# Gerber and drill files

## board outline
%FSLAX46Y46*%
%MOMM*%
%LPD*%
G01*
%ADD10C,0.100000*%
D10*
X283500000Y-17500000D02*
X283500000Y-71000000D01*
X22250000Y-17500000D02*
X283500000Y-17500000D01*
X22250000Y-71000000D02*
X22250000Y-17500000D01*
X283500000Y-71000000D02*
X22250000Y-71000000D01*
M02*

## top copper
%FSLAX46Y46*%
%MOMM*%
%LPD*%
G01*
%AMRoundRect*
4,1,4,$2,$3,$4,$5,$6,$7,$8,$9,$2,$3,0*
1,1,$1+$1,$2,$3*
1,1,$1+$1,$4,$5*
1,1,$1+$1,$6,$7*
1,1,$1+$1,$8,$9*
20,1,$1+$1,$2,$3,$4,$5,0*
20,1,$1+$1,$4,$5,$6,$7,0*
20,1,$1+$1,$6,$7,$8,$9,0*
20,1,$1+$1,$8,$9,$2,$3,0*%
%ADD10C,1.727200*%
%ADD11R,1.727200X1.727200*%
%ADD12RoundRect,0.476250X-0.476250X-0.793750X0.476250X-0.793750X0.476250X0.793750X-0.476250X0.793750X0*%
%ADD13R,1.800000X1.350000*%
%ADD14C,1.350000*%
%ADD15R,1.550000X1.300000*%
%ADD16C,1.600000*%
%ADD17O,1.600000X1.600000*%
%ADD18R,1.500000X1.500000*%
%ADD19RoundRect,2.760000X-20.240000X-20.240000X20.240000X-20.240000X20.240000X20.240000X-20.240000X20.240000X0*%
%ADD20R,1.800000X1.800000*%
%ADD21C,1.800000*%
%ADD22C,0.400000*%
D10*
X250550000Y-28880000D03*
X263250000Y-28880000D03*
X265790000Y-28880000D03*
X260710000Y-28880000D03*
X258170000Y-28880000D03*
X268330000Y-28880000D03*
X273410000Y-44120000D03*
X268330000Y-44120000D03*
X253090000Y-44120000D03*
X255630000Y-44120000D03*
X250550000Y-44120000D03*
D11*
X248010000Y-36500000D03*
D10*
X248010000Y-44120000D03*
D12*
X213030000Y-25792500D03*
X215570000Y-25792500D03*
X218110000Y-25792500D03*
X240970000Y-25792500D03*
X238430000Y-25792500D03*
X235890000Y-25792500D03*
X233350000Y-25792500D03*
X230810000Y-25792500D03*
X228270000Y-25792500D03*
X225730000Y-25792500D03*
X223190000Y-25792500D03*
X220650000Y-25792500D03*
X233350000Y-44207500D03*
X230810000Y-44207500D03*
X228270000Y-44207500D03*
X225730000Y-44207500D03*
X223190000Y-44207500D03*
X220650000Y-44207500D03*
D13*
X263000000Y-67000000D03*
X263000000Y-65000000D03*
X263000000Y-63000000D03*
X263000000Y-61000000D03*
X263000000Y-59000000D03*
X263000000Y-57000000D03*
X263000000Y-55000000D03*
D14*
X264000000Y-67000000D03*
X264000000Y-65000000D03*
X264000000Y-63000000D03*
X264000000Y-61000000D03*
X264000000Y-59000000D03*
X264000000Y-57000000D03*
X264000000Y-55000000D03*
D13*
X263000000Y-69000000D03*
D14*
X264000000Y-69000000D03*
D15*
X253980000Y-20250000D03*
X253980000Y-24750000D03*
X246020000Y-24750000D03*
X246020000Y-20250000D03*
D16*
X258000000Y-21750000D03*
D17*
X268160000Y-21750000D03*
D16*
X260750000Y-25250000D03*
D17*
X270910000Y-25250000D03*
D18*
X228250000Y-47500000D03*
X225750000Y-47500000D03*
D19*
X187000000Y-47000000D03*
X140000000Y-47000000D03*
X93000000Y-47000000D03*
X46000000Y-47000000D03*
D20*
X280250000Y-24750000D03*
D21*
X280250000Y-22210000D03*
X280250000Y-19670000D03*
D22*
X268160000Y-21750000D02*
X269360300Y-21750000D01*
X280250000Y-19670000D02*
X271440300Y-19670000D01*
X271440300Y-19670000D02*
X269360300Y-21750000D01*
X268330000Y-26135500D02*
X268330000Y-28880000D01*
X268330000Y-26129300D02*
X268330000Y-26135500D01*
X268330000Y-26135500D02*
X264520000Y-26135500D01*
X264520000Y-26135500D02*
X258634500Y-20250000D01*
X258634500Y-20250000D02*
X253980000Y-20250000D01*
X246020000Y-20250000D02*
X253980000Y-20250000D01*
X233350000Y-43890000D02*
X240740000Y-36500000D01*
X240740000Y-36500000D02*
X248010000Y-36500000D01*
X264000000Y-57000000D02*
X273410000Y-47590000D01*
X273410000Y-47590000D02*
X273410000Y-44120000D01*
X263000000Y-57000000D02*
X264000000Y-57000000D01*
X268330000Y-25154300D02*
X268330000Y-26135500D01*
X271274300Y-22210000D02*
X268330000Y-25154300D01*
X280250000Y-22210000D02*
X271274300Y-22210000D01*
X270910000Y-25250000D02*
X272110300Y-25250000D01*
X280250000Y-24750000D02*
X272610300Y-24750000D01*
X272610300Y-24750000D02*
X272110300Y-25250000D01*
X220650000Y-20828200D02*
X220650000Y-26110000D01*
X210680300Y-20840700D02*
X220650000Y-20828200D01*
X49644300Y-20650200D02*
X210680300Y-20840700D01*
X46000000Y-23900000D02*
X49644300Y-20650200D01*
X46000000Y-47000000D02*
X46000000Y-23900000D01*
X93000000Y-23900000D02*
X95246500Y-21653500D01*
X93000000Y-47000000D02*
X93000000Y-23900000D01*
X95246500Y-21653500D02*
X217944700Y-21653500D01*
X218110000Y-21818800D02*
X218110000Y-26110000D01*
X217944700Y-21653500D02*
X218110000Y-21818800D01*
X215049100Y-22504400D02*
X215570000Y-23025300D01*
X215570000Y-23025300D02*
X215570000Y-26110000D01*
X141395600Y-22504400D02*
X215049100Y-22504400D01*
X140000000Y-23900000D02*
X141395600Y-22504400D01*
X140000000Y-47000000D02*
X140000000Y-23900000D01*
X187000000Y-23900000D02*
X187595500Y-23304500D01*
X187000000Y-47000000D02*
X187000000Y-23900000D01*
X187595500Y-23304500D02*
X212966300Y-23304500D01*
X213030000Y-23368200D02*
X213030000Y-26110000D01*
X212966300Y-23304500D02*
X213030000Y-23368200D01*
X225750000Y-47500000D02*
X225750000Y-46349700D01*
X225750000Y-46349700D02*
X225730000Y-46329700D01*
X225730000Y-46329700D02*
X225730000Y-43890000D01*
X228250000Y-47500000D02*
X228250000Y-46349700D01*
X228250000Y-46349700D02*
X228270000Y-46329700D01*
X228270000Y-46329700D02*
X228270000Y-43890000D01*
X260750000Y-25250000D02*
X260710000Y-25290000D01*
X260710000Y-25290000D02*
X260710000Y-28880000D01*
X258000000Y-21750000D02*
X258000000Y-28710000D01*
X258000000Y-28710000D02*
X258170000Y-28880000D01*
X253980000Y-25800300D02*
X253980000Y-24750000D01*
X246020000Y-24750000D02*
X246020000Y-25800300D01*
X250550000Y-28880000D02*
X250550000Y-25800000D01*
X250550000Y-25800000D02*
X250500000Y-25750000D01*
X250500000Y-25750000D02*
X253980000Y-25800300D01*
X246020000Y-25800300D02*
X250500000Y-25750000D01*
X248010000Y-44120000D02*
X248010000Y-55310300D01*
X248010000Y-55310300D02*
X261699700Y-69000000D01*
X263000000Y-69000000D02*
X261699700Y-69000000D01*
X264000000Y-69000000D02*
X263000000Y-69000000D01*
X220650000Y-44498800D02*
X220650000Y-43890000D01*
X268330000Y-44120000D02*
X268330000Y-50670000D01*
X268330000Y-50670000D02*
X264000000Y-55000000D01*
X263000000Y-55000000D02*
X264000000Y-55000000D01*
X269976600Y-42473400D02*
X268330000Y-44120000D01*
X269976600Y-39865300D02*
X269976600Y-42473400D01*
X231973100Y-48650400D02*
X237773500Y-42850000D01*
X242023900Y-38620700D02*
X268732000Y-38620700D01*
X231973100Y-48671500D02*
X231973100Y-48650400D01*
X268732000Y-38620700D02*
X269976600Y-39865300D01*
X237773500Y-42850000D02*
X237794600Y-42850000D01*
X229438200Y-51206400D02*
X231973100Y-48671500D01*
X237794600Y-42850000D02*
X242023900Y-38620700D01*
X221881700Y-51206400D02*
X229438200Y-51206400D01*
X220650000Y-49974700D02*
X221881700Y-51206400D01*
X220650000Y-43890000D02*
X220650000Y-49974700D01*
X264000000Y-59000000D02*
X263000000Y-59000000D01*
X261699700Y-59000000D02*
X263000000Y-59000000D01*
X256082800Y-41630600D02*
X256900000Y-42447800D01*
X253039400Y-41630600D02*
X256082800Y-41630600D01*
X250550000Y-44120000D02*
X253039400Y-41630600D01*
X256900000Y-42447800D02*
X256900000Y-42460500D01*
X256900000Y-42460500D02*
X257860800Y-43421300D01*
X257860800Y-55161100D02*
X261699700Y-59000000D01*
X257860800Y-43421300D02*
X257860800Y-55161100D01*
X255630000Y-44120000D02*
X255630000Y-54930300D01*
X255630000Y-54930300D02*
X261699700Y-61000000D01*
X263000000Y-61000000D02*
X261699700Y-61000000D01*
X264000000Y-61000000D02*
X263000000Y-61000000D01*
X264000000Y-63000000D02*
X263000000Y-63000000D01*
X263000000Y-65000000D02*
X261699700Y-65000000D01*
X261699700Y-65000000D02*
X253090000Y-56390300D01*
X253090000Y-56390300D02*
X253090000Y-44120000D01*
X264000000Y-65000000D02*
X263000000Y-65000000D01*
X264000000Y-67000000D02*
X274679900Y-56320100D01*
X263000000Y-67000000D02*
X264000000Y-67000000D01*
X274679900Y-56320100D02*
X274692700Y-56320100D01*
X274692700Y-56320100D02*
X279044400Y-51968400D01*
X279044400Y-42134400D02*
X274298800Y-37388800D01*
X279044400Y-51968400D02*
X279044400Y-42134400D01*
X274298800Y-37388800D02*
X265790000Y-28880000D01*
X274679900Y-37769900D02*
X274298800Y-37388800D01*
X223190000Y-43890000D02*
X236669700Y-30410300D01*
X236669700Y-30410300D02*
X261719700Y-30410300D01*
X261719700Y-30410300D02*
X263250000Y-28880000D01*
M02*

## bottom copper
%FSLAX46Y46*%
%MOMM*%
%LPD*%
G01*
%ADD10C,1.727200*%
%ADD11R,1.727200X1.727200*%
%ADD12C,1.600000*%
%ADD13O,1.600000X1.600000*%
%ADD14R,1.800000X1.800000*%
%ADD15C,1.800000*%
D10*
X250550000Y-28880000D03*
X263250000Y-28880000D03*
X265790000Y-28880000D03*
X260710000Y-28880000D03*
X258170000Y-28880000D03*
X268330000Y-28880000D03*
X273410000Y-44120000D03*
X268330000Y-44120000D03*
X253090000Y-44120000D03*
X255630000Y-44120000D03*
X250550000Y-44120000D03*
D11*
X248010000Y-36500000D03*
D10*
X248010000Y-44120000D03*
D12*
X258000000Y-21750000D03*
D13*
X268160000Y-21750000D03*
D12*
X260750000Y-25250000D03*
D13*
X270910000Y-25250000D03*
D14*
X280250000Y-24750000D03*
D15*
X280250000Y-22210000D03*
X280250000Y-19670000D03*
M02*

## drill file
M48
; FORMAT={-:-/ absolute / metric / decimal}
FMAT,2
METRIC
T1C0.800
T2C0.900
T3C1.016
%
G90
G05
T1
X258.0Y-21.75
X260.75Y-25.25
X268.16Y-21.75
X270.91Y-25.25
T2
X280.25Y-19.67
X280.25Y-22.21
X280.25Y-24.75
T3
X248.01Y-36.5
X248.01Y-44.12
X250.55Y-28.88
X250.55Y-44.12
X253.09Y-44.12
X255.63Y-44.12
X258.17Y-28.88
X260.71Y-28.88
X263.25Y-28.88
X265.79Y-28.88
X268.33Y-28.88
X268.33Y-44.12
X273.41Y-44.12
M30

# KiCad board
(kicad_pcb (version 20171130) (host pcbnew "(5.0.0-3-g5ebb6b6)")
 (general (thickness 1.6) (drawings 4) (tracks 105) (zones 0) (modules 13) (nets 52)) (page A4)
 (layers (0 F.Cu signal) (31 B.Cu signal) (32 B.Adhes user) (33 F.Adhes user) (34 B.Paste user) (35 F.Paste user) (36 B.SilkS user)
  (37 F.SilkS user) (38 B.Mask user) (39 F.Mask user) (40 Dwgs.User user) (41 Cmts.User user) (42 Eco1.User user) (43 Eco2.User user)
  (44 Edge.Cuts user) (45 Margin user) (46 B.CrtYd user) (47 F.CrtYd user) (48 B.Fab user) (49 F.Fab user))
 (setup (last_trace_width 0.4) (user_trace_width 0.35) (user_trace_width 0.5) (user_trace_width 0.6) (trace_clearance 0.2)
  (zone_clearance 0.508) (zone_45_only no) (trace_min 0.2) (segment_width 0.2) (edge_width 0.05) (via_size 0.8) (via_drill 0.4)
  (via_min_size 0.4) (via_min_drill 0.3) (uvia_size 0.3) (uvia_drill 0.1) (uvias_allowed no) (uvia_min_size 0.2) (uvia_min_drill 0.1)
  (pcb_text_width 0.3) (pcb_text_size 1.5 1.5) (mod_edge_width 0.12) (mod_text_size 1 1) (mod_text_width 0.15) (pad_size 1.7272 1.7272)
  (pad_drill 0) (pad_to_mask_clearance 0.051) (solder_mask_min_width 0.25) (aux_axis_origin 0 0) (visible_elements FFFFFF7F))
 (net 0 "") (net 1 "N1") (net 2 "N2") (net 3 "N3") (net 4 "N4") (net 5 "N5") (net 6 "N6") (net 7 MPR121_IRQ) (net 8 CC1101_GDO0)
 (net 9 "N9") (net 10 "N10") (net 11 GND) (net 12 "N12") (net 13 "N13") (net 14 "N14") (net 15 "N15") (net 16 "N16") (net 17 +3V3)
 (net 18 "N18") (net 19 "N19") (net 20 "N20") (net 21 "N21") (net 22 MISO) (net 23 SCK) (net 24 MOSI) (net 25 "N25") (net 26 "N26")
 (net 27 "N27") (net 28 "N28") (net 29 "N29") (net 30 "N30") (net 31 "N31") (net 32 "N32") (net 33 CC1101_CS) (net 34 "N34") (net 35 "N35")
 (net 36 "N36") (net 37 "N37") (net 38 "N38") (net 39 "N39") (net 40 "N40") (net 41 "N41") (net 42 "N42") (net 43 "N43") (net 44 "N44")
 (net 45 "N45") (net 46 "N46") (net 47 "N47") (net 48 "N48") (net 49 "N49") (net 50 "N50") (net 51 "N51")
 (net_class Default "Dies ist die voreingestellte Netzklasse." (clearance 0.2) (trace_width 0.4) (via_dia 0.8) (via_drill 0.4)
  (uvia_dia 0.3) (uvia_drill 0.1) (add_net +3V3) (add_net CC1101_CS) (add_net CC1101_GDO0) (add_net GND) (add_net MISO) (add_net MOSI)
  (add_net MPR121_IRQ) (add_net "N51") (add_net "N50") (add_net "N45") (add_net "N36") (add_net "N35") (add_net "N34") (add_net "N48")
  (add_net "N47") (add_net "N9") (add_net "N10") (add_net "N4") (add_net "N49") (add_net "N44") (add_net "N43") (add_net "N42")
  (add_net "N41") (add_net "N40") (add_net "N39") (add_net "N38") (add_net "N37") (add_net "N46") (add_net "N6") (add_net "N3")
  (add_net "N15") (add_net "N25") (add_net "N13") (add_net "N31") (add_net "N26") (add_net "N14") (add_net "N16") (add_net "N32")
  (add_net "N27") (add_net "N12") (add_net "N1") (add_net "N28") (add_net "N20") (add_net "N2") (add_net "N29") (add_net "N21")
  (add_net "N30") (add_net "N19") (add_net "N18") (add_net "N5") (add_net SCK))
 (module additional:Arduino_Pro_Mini (layer F.Cu) (at 263.25 36.5 270)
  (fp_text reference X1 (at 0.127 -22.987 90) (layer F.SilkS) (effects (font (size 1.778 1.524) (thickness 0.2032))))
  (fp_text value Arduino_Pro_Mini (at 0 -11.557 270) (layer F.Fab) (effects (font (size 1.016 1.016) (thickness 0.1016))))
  (pad 4B connect circle (at 5.08 -1.27 270) (size 1.7272 1.7272) (layers F.Mask) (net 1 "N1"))
  (pad 5B connect circle (at 5.08 -3.81 270) (size 1.7272 1.7272) (layers F.Mask) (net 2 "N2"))
  (pad 12D connect circle (at -7.62 15.24 270) (size 1.7272 1.7272) (layers F.Mask) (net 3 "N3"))
  (pad 11D thru_hole circle (at -7.62 12.7 270) (size 1.7272 1.7272) (drill 1.016) (layers *.Cu *.Mask F.SilkS) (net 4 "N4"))
  (pad 9D connect circle (at -7.62 7.62 270) (size 1.7272 1.7272) (layers F.Mask) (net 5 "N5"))
  (pad 10D connect circle (at -7.62 10.16 270) (size 1.7272 1.7272) (layers F.Mask) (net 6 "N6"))
  (pad 6D thru_hole circle (at -7.62 0 270) (size 1.7272 1.7272) (drill 1.016) (layers *.Cu *.Mask F.SilkS) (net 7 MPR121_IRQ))
  (pad 5D thru_hole circle (at -7.62 -2.54 270) (size 1.7272 1.7272) (drill 1.016) (layers *.Cu *.Mask F.SilkS) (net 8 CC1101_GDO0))
  (pad 7D thru_hole circle (at -7.62 2.54 270) (size 1.7272 1.7272) (drill 1.016) (layers *.Cu *.Mask F.SilkS) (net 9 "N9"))
  (pad 8D thru_hole circle (at -7.62 5.08 270) (size 1.7272 1.7272) (drill 1.016) (layers *.Cu *.Mask F.SilkS) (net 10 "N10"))
  (pad 4D thru_hole circle (at -7.62 -5.08 270) (size 1.7272 1.7272) (drill 1.016) (layers *.Cu *.Mask F.SilkS) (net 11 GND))
  (pad 3D connect circle (at -7.62 -7.62 270) (size 1.7272 1.7272) (layers F.Mask) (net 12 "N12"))
  (pad 1D connect rect (at -7.62 -12.7 270) (size 1.7272 1.7272) (layers F.Mask) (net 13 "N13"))
  (pad 2D connect circle (at -7.62 -10.16 270) (size 1.7272 1.7272) (layers F.Mask) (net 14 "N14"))
  (pad 2A thru_hole circle (at 7.62 -10.16 270) (size 1.7272 1.7272) (drill 1.016) (layers *.Cu *.Mask F.SilkS) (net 11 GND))
  (pad 1A connect rect (at 7.62 -12.7 270) (size 1.7272 1.7272) (layers F.Mask) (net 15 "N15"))
  (pad 3A connect circle (at 7.62 -7.62 270) (size 1.7272 1.7272) (layers F.Mask) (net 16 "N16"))
  (pad 4A thru_hole circle (at 7.62 -5.08 270) (size 1.7272 1.7272) (drill 1.016) (layers *.Cu *.Mask F.SilkS) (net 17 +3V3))
  (pad 8A connect circle (at 7.62 5.08 270) (size 1.7272 1.7272) (layers F.Mask) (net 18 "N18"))
  (pad 7A connect circle (at 7.62 2.54 270) (size 1.7272 1.7272) (layers F.Mask) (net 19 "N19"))
  (pad 5A connect circle (at 7.62 -2.54 270) (size 1.7272 1.7272) (layers F.Mask) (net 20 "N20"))
  (pad 6A connect circle (at 7.62 0 270) (size 1.7272 1.7272) (layers F.Mask) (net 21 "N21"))
  (pad 10A thru_hole circle (at 7.62 10.16 270) (size 1.7272 1.7272) (drill 1.016) (layers *.Cu *.Mask F.SilkS) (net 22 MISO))
  (pad 9A thru_hole circle (at 7.62 7.62 270) (size 1.7272 1.7272) (drill 1.016) (layers *.Cu *.Mask F.SilkS) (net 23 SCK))
  (pad 11A thru_hole circle (at 7.62 12.7 270) (size 1.7272 1.7272) (drill 1.016) (layers *.Cu *.Mask F.SilkS) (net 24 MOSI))
  (pad 1C connect rect (at -6.35 -15.24 270) (size 1.7272 1.7272) (layers F.Mask) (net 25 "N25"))
  (pad 2C connect circle (at -3.81 -15.24 270) (size 1.7272 1.7272) (layers F.Mask) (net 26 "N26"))
  (pad 3C connect circle (at -1.27 -15.24 270) (size 1.7272 1.7272) (layers F.Mask) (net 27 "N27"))
  (pad 4C connect circle (at 1.27 -15.24 270) (size 1.7272 1.7272) (layers F.Mask) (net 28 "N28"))
  (pad 5C connect circle (at 3.81 -15.24 270) (size 1.7272 1.7272) (layers F.Mask) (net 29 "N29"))
  (pad 6C connect circle (at 6.35 -15.24 270) (size 1.7272 1.7272) (layers F.Mask) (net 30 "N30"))
  (pad 1B thru_hole rect (at 0 15.24 270) (size 1.7272 1.7272) (drill 1.016) (layers *.Cu *.Mask F.SilkS) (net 11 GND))
  (pad 2B connect circle (at 2.54 15.24 270) (size 1.7272 1.7272) (layers F.Mask) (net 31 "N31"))
  (pad 3B connect circle (at 5.08 15.24 270) (size 1.7272 1.7272) (layers F.Mask) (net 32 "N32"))
  (pad 12A thru_hole circle (at 7.62 15.24 270) (size 1.7272 1.7272) (drill 1.016) (layers *.Cu *.Mask F.SilkS) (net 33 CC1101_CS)))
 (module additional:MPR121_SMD (layer F.Cu) (at 227 35)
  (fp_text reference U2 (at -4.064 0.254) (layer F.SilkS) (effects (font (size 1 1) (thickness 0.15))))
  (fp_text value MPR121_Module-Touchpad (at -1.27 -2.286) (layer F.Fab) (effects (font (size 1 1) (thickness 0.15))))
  (pad 7 smd roundrect (at -13.97 -8.89) (size 1.905 2.54) (drill oval (offset 0 -0.3175)) (layers F.Cu F.Paste F.Mask)
   (roundrect_rratio 0.25) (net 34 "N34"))
  (pad 8 smd roundrect (at -11.43 -8.89) (size 1.905 2.54) (drill oval (offset 0 -0.3175)) (layers F.Cu F.Paste F.Mask)
   (roundrect_rratio 0.25) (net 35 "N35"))
  (pad 9 smd roundrect (at -8.89 -8.89) (size 1.905 2.54) (drill oval (offset 0 -0.3175)) (layers F.Cu F.Paste F.Mask)
   (roundrect_rratio 0.25) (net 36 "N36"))
  (pad 18 smd roundrect (at 13.97 -8.89) (size 1.905 2.54) (drill oval (offset 0 -0.3175)) (layers F.Cu F.Paste F.Mask)
   (roundrect_rratio 0.25) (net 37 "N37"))
  (pad 17 smd roundrect (at 11.43 -8.89) (size 1.905 2.54) (drill oval (offset 0 -0.3175)) (layers F.Cu F.Paste F.Mask)
   (roundrect_rratio 0.25) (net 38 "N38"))
  (pad 16 smd roundrect (at 8.89 -8.89) (size 1.905 2.54) (drill oval (offset 0 -0.3175)) (layers F.Cu F.Paste F.Mask)
   (roundrect_rratio 0.25) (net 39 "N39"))
  (pad 15 smd roundrect (at 6.35 -8.89) (size 1.905 2.54) (drill oval (offset 0 -0.3175)) (layers F.Cu F.Paste F.Mask)
   (roundrect_rratio 0.25) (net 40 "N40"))
  (pad 14 smd roundrect (at 3.81 -8.89) (size 1.905 2.54) (drill oval (offset 0 -0.3175)) (layers F.Cu F.Paste F.Mask)
   (roundrect_rratio 0.25) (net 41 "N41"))
  (pad 13 smd roundrect (at 1.27 -8.89) (size 1.905 2.54) (drill oval (offset 0 -0.3175)) (layers F.Cu F.Paste F.Mask)
   (roundrect_rratio 0.25) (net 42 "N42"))
  (pad 12 smd roundrect (at -1.27 -8.89) (size 1.905 2.54) (drill oval (offset 0 -0.3175)) (layers F.Cu F.Paste F.Mask)
   (roundrect_rratio 0.25) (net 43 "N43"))
  (pad 11 smd roundrect (at -3.81 -8.89) (size 1.905 2.54) (drill oval (offset 0 -0.3175)) (layers F.Cu F.Paste F.Mask)
   (roundrect_rratio 0.25) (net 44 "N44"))
  (pad 10 smd roundrect (at -6.35 -8.89) (size 1.905 2.54) (drill oval (offset 0 -0.3175)) (layers F.Cu F.Paste F.Mask)
   (roundrect_rratio 0.25) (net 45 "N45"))
  (pad 6 smd roundrect (at 6.35 8.89) (size 1.905 2.54) (drill oval (offset 0 0.3175)) (layers F.Cu F.Paste F.Mask) (roundrect_rratio 0.25)
   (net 11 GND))
  (pad 5 smd roundrect (at 3.81 8.89) (size 1.905 2.54) (drill oval (offset 0 0.3175)) (layers F.Cu F.Paste F.Mask) (roundrect_rratio 0.25)
   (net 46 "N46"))
  (pad 4 smd roundrect (at 1.27 8.89) (size 1.905 2.54) (drill oval (offset 0 0.3175)) (layers F.Cu F.Paste F.Mask) (roundrect_rratio 0.25)
   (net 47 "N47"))
  (pad 3 smd roundrect (at -1.27 8.89) (size 1.905 2.54) (drill oval (offset 0 0.3175)) (layers F.Cu F.Paste F.Mask) (roundrect_rratio 0.25)
   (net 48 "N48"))
  (pad 2 smd roundrect (at -3.81 8.89) (size 1.905 2.54) (drill oval (offset 0 0.3175)) (layers F.Cu F.Paste F.Mask) (roundrect_rratio 0.25)
   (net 7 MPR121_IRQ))
  (pad 1 smd roundrect (at -6.35 8.89) (size 1.905 2.54) (drill oval (offset 0 0.3175)) (layers F.Cu F.Paste F.Mask) (roundrect_rratio 0.25)
   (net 17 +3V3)))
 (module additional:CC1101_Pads (layer F.Cu) (at 261.5 53.5)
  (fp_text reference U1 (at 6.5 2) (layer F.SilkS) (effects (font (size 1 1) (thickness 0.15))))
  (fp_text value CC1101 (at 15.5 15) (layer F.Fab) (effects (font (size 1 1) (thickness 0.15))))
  (pad 7 connect rect (at 1.5 13.5) (size 1.8 1.35) (layers F.Cu F.Mask) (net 8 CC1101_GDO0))
  (pad 6 connect rect (at 1.5 11.5) (size 1.8 1.35) (layers F.Cu F.Mask) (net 22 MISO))
  (pad 5 connect rect (at 1.5 9.5) (size 1.8 1.35) (layers F.Cu F.Mask) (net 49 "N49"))
  (pad 4 connect rect (at 1.5 7.5) (size 1.8 1.35) (layers F.Cu F.Mask) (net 23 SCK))
  (pad 3 connect rect (at 1.5 5.5) (size 1.8 1.35) (layers F.Cu F.Mask) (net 24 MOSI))
  (pad 2 connect rect (at 1.5 3.5) (size 1.8 1.35) (layers F.Cu F.Mask) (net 11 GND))
  (pad 1 connect rect (at 1.5 1.5) (size 1.8 1.35) (layers F.Cu F.Mask) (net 17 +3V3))
  (pad 7 smd circle (at 2.5 13.5) (size 1.35 1.35) (layers F.Cu F.Paste F.Mask) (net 8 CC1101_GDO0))
  (pad 6 smd circle (at 2.5 11.5) (size 1.35 1.35) (layers F.Cu F.Paste F.Mask) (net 22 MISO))
  (pad 5 smd circle (at 2.5 9.5) (size 1.35 1.35) (layers F.Cu F.Paste F.Mask) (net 49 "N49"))
  (pad 4 smd circle (at 2.5 7.5) (size 1.35 1.35) (layers F.Cu F.Paste F.Mask) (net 23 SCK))
  (pad 3 smd circle (at 2.5 5.5) (size 1.35 1.35) (layers F.Cu F.Paste F.Mask) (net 24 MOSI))
  (pad 2 smd circle (at 2.5 3.5) (size 1.35 1.35) (layers F.Cu F.Paste F.Mask) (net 11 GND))
  (pad 1 smd circle (at 2.5 1.5) (size 1.35 1.35) (layers F.Cu F.Paste F.Mask) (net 17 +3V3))
  (pad 8 connect rect (at 1.5 15.5) (size 1.8 1.35) (layers F.Cu F.Mask) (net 33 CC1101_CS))
  (pad 8 smd circle (at 2.5 15.5) (size 1.35 1.35) (layers F.Cu F.Paste F.Mask) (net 33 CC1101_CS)))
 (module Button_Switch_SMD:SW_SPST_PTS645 (layer F.Cu) (at 250 22.5 180)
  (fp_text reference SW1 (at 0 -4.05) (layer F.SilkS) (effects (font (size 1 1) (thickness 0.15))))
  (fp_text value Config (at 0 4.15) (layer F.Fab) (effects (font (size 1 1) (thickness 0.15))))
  (pad 2 smd rect (at -3.98 2.25 180) (size 1.55 1.3) (layers F.Cu F.Paste F.Mask) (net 11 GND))
  (pad 1 smd rect (at -3.98 -2.25 180) (size 1.55 1.3) (layers F.Cu F.Paste F.Mask) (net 4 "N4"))
  (pad 1 smd rect (at 3.98 -2.25 180) (size 1.55 1.3) (layers F.Cu F.Paste F.Mask) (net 4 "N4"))
  (pad 2 smd rect (at 3.98 2.25 180) (size 1.55 1.3) (layers F.Cu F.Paste F.Mask) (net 11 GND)))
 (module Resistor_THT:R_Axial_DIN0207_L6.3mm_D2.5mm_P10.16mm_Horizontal (layer F.Cu) (at 258 21.75)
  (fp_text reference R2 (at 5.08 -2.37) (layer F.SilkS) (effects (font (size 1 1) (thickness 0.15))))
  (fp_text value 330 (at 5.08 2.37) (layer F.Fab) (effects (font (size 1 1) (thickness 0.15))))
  (pad 1 thru_hole circle (at 0 0) (size 1.6 1.6) (drill 0.8) (layers *.Cu *.Mask) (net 10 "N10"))
  (pad 2 thru_hole oval (at 10.16 0) (size 1.6 1.6) (drill 0.8) (layers *.Cu *.Mask) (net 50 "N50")))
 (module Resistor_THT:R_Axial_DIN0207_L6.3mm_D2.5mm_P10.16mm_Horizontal (layer F.Cu) (at 260.75 25.25)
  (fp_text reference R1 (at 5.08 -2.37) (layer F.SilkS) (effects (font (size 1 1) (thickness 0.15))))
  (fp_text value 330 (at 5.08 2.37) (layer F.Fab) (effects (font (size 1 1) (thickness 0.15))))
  (pad 1 thru_hole circle (at 0 0) (size 1.6 1.6) (drill 0.8) (layers *.Cu *.Mask) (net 9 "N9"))
  (pad 2 thru_hole oval (at 10.16 0) (size 1.6 1.6) (drill 0.8) (layers *.Cu *.Mask) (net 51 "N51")))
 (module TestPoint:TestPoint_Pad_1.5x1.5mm (layer F.Cu) (at 228.25 47.5)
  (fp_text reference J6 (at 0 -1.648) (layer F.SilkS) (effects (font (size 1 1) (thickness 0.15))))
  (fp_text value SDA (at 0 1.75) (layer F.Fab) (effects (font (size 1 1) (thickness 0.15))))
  (pad 1 smd rect (at 0 0) (size 1.5 1.5) (layers F.Cu F.Mask) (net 47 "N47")))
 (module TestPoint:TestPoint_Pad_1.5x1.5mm (layer F.Cu) (at 225.75 47.5)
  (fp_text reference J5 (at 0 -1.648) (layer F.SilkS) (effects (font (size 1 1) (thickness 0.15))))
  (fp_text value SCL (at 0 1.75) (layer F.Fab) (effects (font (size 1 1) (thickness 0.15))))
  (pad 1 smd rect (at 0 0) (size 1.5 1.5) (layers F.Cu F.Mask) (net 48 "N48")))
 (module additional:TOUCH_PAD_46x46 (layer F.Cu) (at 187 47)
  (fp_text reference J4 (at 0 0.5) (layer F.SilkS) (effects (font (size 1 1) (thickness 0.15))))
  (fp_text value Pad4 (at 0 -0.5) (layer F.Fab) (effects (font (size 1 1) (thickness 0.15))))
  (pad 1 smd roundrect (at 0 0) (size 46 46) (layers F.Cu) (roundrect_rratio 0.06) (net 34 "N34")))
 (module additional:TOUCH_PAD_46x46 (layer F.Cu) (at 140 47)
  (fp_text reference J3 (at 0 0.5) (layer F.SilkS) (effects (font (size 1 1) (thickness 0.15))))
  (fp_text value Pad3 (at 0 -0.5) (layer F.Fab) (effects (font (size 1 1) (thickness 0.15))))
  (pad 1 smd roundrect (at 0 0) (size 46 46) (layers F.Cu) (roundrect_rratio 0.06) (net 35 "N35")))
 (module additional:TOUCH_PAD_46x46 (layer F.Cu) (at 93 47)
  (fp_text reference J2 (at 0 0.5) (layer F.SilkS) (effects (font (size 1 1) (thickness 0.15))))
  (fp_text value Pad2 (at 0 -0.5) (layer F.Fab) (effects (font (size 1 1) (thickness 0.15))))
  (pad 1 smd roundrect (at 0 0) (size 46 46) (layers F.Cu) (roundrect_rratio 0.06) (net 36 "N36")))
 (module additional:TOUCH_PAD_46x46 (layer F.Cu) (at 46 47)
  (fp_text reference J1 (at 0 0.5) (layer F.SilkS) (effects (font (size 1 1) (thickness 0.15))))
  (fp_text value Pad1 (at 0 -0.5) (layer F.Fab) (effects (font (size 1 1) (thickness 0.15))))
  (pad 1 smd roundrect (at 0 0) (size 46 46) (layers F.Cu) (roundrect_rratio 0.06) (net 45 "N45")))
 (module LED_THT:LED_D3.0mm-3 (layer F.Cu) (at 280.25 24.75 90)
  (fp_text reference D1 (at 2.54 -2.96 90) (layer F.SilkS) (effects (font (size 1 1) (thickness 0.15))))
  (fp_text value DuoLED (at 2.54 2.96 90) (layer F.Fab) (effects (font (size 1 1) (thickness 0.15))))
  (pad 1 thru_hole rect (at 0 0 90) (size 1.8 1.8) (drill 0.9) (layers *.Cu *.Mask) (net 51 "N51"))
  (pad 2 thru_hole circle (at 2.54 0 90) (size 1.8 1.8) (drill 0.9) (layers *.Cu *.Mask) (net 11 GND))
  (pad 3 thru_hole circle (at 5.08 0 90) (size 1.8 1.8) (drill 0.9) (layers *.Cu *.Mask) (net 50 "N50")))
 (gr_line (start 283.5 17.5) (end 283.5 71) (layer Edge.Cuts) (width 0.1))
 (gr_line (start 22.25 17.5) (end 283.5 17.5) (layer Edge.Cuts) (width 0.1))
 (gr_line (start 22.25 71) (end 22.25 17.5) (layer Edge.Cuts) (width 0.1))
 (gr_line (start 283.5 71) (end 22.25 71) (layer Edge.Cuts) (width 0.1))
 (segment (start 268.16 21.75) (end 269.3603 21.75) (width 0.4) (layer F.Cu) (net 50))
 (segment (start 280.25 19.67) (end 271.4403 19.67) (width 0.4) (layer F.Cu) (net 50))
 (segment (start 271.4403 19.67) (end 269.3603 21.75) (width 0.4) (layer F.Cu) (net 50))
 (segment (start 268.33 26.1355) (end 268.33 28.88) (width 0.4) (layer F.Cu) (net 11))
 (segment (start 268.33 26.1293) (end 268.33 26.1355) (width 0.4) (layer F.Cu) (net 11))
 (segment (start 268.33 26.1355) (end 264.52 26.1355) (width 0.4) (layer F.Cu) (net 11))
 (segment (start 264.52 26.1355) (end 258.6345 20.25) (width 0.4) (layer F.Cu) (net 11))
 (segment (start 258.6345 20.25) (end 253.98 20.25) (width 0.4) (layer F.Cu) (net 11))
 (segment (start 246.02 20.25) (end 253.98 20.25) (width 0.4) (layer F.Cu) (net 11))
 (segment (start 233.35 43.89) (end 240.74 36.5) (width 0.4) (layer F.Cu) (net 11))
 (segment (start 240.74 36.5) (end 248.01 36.5) (width 0.4) (layer F.Cu) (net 11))
 (segment (start 264 57) (end 273.41 47.59) (width 0.4) (layer F.Cu) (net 11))
 (segment (start 273.41 47.59) (end 273.41 44.12) (width 0.4) (layer F.Cu) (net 11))
 (segment (start 263 57) (end 264 57) (width 0.4) (layer F.Cu) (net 11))
 (segment (start 268.33 25.1543) (end 268.33 26.1355) (width 0.4) (layer F.Cu) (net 11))
 (segment (start 271.2743 22.21) (end 268.33 25.1543) (width 0.4) (layer F.Cu) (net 11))
 (segment (start 280.25 22.21) (end 271.2743 22.21) (width 0.4) (layer F.Cu) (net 11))
 (segment (start 270.91 25.25) (end 272.1103 25.25) (width 0.4) (layer F.Cu) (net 51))
 (segment (start 280.25 24.75) (end 272.6103 24.75) (width 0.4) (layer F.Cu) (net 51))
 (segment (start 272.6103 24.75) (end 272.1103 25.25) (width 0.4) (layer F.Cu) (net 51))
 (segment (start 220.65 20.8282) (end 220.65 26.11) (width 0.4) (layer F.Cu) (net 45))
 (segment (start 210.6803 20.8407) (end 220.65 20.8282) (width 0.4) (layer F.Cu) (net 45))
 (segment (start 49.6443 20.6502) (end 210.6803 20.8407) (width 0.4) (layer F.Cu) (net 45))
 (segment (start 46 23.9) (end 49.6443 20.6502) (width 0.4) (layer F.Cu) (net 45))
 (segment (start 46 47) (end 46 23.9) (width 0.4) (layer F.Cu) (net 45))
 (segment (start 93 23.9) (end 95.2465 21.6535) (width 0.4) (layer F.Cu) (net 36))
 (segment (start 93 47) (end 93 23.9) (width 0.4) (layer F.Cu) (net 36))
 (segment (start 95.2465 21.6535) (end 217.9447 21.6535) (width 0.4) (layer F.Cu) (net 36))
 (segment (start 218.11 21.8188) (end 218.11 26.11) (width 0.4) (layer F.Cu) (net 36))
 (segment (start 217.9447 21.6535) (end 218.11 21.8188) (width 0.4) (layer F.Cu) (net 36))
 (segment (start 215.0491 22.5044) (end 215.57 23.0253) (width 0.4) (layer F.Cu) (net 35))
 (segment (start 215.57 23.0253) (end 215.57 26.11) (width 0.4) (layer F.Cu) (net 35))
 (segment (start 141.3956 22.5044) (end 215.0491 22.5044) (width 0.4) (layer F.Cu) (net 35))
 (segment (start 140 23.9) (end 141.3956 22.5044) (width 0.4) (layer F.Cu) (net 35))
 (segment (start 140 47) (end 140 23.9) (width 0.4) (layer F.Cu) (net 35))
 (segment (start 187 23.9) (end 187.5955 23.3045) (width 0.4) (layer F.Cu) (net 34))
 (segment (start 187 47) (end 187 23.9) (width 0.4) (layer F.Cu) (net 34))
 (segment (start 187.5955 23.3045) (end 212.9663 23.3045) (width 0.4) (layer F.Cu) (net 34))
 (segment (start 213.03 23.3682) (end 213.03 26.11) (width 0.4) (layer F.Cu) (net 34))
 (segment (start 212.9663 23.3045) (end 213.03 23.3682) (width 0.4) (layer F.Cu) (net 34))
 (segment (start 225.75 47.5) (end 225.75 46.3497) (width 0.4) (layer F.Cu) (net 48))
 (segment (start 225.75 46.3497) (end 225.73 46.3297) (width 0.4) (layer F.Cu) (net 48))
 (segment (start 225.73 46.3297) (end 225.73 43.89) (width 0.4) (layer F.Cu) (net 48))
 (segment (start 228.25 47.5) (end 228.25 46.3497) (width 0.4) (layer F.Cu) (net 47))
 (segment (start 228.25 46.3497) (end 228.27 46.3297) (width 0.4) (layer F.Cu) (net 47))
 (segment (start 228.27 46.3297) (end 228.27 43.89) (width 0.4) (layer F.Cu) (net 47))
 (segment (start 260.75 25.25) (end 260.71 25.29) (width 0.4) (layer F.Cu) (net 9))
 (segment (start 260.71 25.29) (end 260.71 28.88) (width 0.4) (layer F.Cu) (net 9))
 (segment (start 258 21.75) (end 258 28.71) (width 0.4) (layer F.Cu) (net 10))
 (segment (start 258 28.71) (end 258.17 28.88) (width 0.4) (layer F.Cu) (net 10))
 (segment (start 253.98 25.8003) (end 253.98 24.75) (width 0.4) (layer F.Cu) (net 4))
 (segment (start 246.02 24.75) (end 246.02 25.8003) (width 0.4) (layer F.Cu) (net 4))
 (segment (start 250.55 28.88) (end 250.55 25.8) (width 0.4) (layer F.Cu) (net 4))
 (segment (start 250.55 25.8) (end 250.5 25.75) (width 0.4) (layer F.Cu) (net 4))
 (segment (start 250.5 25.75) (end 253.98 25.8003) (width 0.4) (layer F.Cu) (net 4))
 (segment (start 246.02 25.8003) (end 250.5 25.75) (width 0.4) (layer F.Cu) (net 4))
 (segment (start 248.01 44.12) (end 248.01 55.3103) (width 0.4) (layer F.Cu) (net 33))
 (segment (start 248.01 55.3103) (end 261.6997 69) (width 0.4) (layer F.Cu) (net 33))
 (segment (start 263 69) (end 261.6997 69) (width 0.4) (layer F.Cu) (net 33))
 (segment (start 264 69) (end 263 69) (width 0.4) (layer F.Cu) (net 33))
 (segment (start 220.65 44.4988) (end 220.65 43.89) (width 0.4) (layer F.Cu) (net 17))
 (segment (start 268.33 44.12) (end 268.33 50.67) (width 0.4) (layer F.Cu) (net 17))
 (segment (start 268.33 50.67) (end 264 55) (width 0.4) (layer F.Cu) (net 17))
 (segment (start 263 55) (end 264 55) (width 0.4) (layer F.Cu) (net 17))
 (segment (start 269.9766 42.4734) (end 268.33 44.12) (width 0.4) (layer F.Cu) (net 17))
 (segment (start 269.9766 39.8653) (end 269.9766 42.4734) (width 0.4) (layer F.Cu) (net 17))
 (segment (start 231.9731 48.6504) (end 237.7735 42.85) (width 0.4) (layer F.Cu) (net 17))
 (segment (start 242.0239 38.6207) (end 268.732 38.6207) (width 0.4) (layer F.Cu) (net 17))
 (segment (start 231.9731 48.6715) (end 231.9731 48.6504) (width 0.4) (layer F.Cu) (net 17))
 (segment (start 268.732 38.6207) (end 269.9766 39.8653) (width 0.4) (layer F.Cu) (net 17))
 (segment (start 237.7735 42.85) (end 237.7946 42.85) (width 0.4) (layer F.Cu) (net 17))
 (segment (start 229.4382 51.2064) (end 231.9731 48.6715) (width 0.4) (layer F.Cu) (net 17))
 (segment (start 237.7946 42.85) (end 242.0239 38.6207) (width 0.4) (layer F.Cu) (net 17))
 (segment (start 221.8817 51.2064) (end 229.4382 51.2064) (width 0.4) (layer F.Cu) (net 17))
 (segment (start 220.65 49.9747) (end 221.8817 51.2064) (width 0.4) (layer F.Cu) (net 17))
 (segment (start 220.65 43.89) (end 220.65 49.9747) (width 0.4) (layer F.Cu) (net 17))
 (segment (start 264 59) (end 263 59) (width 0.4) (layer F.Cu) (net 24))
 (segment (start 261.6997 59) (end 263 59) (width 0.4) (layer F.Cu) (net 24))
 (segment (start 256.0828 41.6306) (end 256.9 42.4478) (width 0.4) (layer F.Cu) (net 24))
 (segment (start 253.0394 41.6306) (end 256.0828 41.6306) (width 0.4) (layer F.Cu) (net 24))
 (segment (start 250.55 44.12) (end 253.0394 41.6306) (width 0.4) (layer F.Cu) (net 24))
 (segment (start 256.9 42.4478) (end 256.9 42.4605) (width 0.4) (layer F.Cu) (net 24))
 (segment (start 256.9 42.4605) (end 257.8608 43.4213) (width 0.4) (layer F.Cu) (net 24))
 (segment (start 257.8608 55.1611) (end 261.6997 59) (width 0.4) (layer F.Cu) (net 24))
 (segment (start 257.8608 43.4213) (end 257.8608 55.1611) (width 0.4) (layer F.Cu) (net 24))
 (segment (start 255.63 44.12) (end 255.63 54.9303) (width 0.4) (layer F.Cu) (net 23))
 (segment (start 255.63 54.9303) (end 261.6997 61) (width 0.4) (layer F.Cu) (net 23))
 (segment (start 263 61) (end 261.6997 61) (width 0.4) (layer F.Cu) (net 23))
 (segment (start 264 61) (end 263 61) (width 0.4) (layer F.Cu) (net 23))
 (segment (start 264 63) (end 263 63) (width 0.4) (layer F.Cu) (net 49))
 (segment (start 263 65) (end 261.6997 65) (width 0.4) (layer F.Cu) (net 22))
 (segment (start 261.6997 65) (end 253.09 56.3903) (width 0.4) (layer F.Cu) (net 22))
 (segment (start 253.09 56.3903) (end 253.09 44.12) (width 0.4) (layer F.Cu) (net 22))
 (segment (start 264 65) (end 263 65) (width 0.4) (layer F.Cu) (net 22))
 (segment (start 264 67) (end 274.6799 56.3201) (width 0.4) (layer F.Cu) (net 8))
 (segment (start 263 67) (end 264 67) (width 0.4) (layer F.Cu) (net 8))
 (segment (start 274.6799 56.3201) (end 274.6927 56.3201) (width 0.4) (layer F.Cu) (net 8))
 (segment (start 274.6927 56.3201) (end 279.0444 51.9684) (width 0.4) (layer F.Cu) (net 8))
 (segment (start 279.0444 42.1344) (end 274.2988 37.3888) (width 0.4) (layer F.Cu) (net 8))
 (segment (start 279.0444 51.9684) (end 279.0444 42.1344) (width 0.4) (layer F.Cu) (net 8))
 (segment (start 274.2988 37.3888) (end 265.79 28.88) (width 0.4) (layer F.Cu) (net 8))
 (segment (start 274.6799 37.7699) (end 274.2988 37.3888) (width 0.4) (layer F.Cu) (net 8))
 (segment (start 223.19 43.89) (end 236.6697 30.4103) (width 0.4) (layer F.Cu) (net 7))
 (segment (start 236.6697 30.4103) (end 261.7197 30.4103) (width 0.4) (layer F.Cu) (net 7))
 (segment (start 261.7197 30.4103) (end 263.25 28.88) (width 0.4) (layer F.Cu) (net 7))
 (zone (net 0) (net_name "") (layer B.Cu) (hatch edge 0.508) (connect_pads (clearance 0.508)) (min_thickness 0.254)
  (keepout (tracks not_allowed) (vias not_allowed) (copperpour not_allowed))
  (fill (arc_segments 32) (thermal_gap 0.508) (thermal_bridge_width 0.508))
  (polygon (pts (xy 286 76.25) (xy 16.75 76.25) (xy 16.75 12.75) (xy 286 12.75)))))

